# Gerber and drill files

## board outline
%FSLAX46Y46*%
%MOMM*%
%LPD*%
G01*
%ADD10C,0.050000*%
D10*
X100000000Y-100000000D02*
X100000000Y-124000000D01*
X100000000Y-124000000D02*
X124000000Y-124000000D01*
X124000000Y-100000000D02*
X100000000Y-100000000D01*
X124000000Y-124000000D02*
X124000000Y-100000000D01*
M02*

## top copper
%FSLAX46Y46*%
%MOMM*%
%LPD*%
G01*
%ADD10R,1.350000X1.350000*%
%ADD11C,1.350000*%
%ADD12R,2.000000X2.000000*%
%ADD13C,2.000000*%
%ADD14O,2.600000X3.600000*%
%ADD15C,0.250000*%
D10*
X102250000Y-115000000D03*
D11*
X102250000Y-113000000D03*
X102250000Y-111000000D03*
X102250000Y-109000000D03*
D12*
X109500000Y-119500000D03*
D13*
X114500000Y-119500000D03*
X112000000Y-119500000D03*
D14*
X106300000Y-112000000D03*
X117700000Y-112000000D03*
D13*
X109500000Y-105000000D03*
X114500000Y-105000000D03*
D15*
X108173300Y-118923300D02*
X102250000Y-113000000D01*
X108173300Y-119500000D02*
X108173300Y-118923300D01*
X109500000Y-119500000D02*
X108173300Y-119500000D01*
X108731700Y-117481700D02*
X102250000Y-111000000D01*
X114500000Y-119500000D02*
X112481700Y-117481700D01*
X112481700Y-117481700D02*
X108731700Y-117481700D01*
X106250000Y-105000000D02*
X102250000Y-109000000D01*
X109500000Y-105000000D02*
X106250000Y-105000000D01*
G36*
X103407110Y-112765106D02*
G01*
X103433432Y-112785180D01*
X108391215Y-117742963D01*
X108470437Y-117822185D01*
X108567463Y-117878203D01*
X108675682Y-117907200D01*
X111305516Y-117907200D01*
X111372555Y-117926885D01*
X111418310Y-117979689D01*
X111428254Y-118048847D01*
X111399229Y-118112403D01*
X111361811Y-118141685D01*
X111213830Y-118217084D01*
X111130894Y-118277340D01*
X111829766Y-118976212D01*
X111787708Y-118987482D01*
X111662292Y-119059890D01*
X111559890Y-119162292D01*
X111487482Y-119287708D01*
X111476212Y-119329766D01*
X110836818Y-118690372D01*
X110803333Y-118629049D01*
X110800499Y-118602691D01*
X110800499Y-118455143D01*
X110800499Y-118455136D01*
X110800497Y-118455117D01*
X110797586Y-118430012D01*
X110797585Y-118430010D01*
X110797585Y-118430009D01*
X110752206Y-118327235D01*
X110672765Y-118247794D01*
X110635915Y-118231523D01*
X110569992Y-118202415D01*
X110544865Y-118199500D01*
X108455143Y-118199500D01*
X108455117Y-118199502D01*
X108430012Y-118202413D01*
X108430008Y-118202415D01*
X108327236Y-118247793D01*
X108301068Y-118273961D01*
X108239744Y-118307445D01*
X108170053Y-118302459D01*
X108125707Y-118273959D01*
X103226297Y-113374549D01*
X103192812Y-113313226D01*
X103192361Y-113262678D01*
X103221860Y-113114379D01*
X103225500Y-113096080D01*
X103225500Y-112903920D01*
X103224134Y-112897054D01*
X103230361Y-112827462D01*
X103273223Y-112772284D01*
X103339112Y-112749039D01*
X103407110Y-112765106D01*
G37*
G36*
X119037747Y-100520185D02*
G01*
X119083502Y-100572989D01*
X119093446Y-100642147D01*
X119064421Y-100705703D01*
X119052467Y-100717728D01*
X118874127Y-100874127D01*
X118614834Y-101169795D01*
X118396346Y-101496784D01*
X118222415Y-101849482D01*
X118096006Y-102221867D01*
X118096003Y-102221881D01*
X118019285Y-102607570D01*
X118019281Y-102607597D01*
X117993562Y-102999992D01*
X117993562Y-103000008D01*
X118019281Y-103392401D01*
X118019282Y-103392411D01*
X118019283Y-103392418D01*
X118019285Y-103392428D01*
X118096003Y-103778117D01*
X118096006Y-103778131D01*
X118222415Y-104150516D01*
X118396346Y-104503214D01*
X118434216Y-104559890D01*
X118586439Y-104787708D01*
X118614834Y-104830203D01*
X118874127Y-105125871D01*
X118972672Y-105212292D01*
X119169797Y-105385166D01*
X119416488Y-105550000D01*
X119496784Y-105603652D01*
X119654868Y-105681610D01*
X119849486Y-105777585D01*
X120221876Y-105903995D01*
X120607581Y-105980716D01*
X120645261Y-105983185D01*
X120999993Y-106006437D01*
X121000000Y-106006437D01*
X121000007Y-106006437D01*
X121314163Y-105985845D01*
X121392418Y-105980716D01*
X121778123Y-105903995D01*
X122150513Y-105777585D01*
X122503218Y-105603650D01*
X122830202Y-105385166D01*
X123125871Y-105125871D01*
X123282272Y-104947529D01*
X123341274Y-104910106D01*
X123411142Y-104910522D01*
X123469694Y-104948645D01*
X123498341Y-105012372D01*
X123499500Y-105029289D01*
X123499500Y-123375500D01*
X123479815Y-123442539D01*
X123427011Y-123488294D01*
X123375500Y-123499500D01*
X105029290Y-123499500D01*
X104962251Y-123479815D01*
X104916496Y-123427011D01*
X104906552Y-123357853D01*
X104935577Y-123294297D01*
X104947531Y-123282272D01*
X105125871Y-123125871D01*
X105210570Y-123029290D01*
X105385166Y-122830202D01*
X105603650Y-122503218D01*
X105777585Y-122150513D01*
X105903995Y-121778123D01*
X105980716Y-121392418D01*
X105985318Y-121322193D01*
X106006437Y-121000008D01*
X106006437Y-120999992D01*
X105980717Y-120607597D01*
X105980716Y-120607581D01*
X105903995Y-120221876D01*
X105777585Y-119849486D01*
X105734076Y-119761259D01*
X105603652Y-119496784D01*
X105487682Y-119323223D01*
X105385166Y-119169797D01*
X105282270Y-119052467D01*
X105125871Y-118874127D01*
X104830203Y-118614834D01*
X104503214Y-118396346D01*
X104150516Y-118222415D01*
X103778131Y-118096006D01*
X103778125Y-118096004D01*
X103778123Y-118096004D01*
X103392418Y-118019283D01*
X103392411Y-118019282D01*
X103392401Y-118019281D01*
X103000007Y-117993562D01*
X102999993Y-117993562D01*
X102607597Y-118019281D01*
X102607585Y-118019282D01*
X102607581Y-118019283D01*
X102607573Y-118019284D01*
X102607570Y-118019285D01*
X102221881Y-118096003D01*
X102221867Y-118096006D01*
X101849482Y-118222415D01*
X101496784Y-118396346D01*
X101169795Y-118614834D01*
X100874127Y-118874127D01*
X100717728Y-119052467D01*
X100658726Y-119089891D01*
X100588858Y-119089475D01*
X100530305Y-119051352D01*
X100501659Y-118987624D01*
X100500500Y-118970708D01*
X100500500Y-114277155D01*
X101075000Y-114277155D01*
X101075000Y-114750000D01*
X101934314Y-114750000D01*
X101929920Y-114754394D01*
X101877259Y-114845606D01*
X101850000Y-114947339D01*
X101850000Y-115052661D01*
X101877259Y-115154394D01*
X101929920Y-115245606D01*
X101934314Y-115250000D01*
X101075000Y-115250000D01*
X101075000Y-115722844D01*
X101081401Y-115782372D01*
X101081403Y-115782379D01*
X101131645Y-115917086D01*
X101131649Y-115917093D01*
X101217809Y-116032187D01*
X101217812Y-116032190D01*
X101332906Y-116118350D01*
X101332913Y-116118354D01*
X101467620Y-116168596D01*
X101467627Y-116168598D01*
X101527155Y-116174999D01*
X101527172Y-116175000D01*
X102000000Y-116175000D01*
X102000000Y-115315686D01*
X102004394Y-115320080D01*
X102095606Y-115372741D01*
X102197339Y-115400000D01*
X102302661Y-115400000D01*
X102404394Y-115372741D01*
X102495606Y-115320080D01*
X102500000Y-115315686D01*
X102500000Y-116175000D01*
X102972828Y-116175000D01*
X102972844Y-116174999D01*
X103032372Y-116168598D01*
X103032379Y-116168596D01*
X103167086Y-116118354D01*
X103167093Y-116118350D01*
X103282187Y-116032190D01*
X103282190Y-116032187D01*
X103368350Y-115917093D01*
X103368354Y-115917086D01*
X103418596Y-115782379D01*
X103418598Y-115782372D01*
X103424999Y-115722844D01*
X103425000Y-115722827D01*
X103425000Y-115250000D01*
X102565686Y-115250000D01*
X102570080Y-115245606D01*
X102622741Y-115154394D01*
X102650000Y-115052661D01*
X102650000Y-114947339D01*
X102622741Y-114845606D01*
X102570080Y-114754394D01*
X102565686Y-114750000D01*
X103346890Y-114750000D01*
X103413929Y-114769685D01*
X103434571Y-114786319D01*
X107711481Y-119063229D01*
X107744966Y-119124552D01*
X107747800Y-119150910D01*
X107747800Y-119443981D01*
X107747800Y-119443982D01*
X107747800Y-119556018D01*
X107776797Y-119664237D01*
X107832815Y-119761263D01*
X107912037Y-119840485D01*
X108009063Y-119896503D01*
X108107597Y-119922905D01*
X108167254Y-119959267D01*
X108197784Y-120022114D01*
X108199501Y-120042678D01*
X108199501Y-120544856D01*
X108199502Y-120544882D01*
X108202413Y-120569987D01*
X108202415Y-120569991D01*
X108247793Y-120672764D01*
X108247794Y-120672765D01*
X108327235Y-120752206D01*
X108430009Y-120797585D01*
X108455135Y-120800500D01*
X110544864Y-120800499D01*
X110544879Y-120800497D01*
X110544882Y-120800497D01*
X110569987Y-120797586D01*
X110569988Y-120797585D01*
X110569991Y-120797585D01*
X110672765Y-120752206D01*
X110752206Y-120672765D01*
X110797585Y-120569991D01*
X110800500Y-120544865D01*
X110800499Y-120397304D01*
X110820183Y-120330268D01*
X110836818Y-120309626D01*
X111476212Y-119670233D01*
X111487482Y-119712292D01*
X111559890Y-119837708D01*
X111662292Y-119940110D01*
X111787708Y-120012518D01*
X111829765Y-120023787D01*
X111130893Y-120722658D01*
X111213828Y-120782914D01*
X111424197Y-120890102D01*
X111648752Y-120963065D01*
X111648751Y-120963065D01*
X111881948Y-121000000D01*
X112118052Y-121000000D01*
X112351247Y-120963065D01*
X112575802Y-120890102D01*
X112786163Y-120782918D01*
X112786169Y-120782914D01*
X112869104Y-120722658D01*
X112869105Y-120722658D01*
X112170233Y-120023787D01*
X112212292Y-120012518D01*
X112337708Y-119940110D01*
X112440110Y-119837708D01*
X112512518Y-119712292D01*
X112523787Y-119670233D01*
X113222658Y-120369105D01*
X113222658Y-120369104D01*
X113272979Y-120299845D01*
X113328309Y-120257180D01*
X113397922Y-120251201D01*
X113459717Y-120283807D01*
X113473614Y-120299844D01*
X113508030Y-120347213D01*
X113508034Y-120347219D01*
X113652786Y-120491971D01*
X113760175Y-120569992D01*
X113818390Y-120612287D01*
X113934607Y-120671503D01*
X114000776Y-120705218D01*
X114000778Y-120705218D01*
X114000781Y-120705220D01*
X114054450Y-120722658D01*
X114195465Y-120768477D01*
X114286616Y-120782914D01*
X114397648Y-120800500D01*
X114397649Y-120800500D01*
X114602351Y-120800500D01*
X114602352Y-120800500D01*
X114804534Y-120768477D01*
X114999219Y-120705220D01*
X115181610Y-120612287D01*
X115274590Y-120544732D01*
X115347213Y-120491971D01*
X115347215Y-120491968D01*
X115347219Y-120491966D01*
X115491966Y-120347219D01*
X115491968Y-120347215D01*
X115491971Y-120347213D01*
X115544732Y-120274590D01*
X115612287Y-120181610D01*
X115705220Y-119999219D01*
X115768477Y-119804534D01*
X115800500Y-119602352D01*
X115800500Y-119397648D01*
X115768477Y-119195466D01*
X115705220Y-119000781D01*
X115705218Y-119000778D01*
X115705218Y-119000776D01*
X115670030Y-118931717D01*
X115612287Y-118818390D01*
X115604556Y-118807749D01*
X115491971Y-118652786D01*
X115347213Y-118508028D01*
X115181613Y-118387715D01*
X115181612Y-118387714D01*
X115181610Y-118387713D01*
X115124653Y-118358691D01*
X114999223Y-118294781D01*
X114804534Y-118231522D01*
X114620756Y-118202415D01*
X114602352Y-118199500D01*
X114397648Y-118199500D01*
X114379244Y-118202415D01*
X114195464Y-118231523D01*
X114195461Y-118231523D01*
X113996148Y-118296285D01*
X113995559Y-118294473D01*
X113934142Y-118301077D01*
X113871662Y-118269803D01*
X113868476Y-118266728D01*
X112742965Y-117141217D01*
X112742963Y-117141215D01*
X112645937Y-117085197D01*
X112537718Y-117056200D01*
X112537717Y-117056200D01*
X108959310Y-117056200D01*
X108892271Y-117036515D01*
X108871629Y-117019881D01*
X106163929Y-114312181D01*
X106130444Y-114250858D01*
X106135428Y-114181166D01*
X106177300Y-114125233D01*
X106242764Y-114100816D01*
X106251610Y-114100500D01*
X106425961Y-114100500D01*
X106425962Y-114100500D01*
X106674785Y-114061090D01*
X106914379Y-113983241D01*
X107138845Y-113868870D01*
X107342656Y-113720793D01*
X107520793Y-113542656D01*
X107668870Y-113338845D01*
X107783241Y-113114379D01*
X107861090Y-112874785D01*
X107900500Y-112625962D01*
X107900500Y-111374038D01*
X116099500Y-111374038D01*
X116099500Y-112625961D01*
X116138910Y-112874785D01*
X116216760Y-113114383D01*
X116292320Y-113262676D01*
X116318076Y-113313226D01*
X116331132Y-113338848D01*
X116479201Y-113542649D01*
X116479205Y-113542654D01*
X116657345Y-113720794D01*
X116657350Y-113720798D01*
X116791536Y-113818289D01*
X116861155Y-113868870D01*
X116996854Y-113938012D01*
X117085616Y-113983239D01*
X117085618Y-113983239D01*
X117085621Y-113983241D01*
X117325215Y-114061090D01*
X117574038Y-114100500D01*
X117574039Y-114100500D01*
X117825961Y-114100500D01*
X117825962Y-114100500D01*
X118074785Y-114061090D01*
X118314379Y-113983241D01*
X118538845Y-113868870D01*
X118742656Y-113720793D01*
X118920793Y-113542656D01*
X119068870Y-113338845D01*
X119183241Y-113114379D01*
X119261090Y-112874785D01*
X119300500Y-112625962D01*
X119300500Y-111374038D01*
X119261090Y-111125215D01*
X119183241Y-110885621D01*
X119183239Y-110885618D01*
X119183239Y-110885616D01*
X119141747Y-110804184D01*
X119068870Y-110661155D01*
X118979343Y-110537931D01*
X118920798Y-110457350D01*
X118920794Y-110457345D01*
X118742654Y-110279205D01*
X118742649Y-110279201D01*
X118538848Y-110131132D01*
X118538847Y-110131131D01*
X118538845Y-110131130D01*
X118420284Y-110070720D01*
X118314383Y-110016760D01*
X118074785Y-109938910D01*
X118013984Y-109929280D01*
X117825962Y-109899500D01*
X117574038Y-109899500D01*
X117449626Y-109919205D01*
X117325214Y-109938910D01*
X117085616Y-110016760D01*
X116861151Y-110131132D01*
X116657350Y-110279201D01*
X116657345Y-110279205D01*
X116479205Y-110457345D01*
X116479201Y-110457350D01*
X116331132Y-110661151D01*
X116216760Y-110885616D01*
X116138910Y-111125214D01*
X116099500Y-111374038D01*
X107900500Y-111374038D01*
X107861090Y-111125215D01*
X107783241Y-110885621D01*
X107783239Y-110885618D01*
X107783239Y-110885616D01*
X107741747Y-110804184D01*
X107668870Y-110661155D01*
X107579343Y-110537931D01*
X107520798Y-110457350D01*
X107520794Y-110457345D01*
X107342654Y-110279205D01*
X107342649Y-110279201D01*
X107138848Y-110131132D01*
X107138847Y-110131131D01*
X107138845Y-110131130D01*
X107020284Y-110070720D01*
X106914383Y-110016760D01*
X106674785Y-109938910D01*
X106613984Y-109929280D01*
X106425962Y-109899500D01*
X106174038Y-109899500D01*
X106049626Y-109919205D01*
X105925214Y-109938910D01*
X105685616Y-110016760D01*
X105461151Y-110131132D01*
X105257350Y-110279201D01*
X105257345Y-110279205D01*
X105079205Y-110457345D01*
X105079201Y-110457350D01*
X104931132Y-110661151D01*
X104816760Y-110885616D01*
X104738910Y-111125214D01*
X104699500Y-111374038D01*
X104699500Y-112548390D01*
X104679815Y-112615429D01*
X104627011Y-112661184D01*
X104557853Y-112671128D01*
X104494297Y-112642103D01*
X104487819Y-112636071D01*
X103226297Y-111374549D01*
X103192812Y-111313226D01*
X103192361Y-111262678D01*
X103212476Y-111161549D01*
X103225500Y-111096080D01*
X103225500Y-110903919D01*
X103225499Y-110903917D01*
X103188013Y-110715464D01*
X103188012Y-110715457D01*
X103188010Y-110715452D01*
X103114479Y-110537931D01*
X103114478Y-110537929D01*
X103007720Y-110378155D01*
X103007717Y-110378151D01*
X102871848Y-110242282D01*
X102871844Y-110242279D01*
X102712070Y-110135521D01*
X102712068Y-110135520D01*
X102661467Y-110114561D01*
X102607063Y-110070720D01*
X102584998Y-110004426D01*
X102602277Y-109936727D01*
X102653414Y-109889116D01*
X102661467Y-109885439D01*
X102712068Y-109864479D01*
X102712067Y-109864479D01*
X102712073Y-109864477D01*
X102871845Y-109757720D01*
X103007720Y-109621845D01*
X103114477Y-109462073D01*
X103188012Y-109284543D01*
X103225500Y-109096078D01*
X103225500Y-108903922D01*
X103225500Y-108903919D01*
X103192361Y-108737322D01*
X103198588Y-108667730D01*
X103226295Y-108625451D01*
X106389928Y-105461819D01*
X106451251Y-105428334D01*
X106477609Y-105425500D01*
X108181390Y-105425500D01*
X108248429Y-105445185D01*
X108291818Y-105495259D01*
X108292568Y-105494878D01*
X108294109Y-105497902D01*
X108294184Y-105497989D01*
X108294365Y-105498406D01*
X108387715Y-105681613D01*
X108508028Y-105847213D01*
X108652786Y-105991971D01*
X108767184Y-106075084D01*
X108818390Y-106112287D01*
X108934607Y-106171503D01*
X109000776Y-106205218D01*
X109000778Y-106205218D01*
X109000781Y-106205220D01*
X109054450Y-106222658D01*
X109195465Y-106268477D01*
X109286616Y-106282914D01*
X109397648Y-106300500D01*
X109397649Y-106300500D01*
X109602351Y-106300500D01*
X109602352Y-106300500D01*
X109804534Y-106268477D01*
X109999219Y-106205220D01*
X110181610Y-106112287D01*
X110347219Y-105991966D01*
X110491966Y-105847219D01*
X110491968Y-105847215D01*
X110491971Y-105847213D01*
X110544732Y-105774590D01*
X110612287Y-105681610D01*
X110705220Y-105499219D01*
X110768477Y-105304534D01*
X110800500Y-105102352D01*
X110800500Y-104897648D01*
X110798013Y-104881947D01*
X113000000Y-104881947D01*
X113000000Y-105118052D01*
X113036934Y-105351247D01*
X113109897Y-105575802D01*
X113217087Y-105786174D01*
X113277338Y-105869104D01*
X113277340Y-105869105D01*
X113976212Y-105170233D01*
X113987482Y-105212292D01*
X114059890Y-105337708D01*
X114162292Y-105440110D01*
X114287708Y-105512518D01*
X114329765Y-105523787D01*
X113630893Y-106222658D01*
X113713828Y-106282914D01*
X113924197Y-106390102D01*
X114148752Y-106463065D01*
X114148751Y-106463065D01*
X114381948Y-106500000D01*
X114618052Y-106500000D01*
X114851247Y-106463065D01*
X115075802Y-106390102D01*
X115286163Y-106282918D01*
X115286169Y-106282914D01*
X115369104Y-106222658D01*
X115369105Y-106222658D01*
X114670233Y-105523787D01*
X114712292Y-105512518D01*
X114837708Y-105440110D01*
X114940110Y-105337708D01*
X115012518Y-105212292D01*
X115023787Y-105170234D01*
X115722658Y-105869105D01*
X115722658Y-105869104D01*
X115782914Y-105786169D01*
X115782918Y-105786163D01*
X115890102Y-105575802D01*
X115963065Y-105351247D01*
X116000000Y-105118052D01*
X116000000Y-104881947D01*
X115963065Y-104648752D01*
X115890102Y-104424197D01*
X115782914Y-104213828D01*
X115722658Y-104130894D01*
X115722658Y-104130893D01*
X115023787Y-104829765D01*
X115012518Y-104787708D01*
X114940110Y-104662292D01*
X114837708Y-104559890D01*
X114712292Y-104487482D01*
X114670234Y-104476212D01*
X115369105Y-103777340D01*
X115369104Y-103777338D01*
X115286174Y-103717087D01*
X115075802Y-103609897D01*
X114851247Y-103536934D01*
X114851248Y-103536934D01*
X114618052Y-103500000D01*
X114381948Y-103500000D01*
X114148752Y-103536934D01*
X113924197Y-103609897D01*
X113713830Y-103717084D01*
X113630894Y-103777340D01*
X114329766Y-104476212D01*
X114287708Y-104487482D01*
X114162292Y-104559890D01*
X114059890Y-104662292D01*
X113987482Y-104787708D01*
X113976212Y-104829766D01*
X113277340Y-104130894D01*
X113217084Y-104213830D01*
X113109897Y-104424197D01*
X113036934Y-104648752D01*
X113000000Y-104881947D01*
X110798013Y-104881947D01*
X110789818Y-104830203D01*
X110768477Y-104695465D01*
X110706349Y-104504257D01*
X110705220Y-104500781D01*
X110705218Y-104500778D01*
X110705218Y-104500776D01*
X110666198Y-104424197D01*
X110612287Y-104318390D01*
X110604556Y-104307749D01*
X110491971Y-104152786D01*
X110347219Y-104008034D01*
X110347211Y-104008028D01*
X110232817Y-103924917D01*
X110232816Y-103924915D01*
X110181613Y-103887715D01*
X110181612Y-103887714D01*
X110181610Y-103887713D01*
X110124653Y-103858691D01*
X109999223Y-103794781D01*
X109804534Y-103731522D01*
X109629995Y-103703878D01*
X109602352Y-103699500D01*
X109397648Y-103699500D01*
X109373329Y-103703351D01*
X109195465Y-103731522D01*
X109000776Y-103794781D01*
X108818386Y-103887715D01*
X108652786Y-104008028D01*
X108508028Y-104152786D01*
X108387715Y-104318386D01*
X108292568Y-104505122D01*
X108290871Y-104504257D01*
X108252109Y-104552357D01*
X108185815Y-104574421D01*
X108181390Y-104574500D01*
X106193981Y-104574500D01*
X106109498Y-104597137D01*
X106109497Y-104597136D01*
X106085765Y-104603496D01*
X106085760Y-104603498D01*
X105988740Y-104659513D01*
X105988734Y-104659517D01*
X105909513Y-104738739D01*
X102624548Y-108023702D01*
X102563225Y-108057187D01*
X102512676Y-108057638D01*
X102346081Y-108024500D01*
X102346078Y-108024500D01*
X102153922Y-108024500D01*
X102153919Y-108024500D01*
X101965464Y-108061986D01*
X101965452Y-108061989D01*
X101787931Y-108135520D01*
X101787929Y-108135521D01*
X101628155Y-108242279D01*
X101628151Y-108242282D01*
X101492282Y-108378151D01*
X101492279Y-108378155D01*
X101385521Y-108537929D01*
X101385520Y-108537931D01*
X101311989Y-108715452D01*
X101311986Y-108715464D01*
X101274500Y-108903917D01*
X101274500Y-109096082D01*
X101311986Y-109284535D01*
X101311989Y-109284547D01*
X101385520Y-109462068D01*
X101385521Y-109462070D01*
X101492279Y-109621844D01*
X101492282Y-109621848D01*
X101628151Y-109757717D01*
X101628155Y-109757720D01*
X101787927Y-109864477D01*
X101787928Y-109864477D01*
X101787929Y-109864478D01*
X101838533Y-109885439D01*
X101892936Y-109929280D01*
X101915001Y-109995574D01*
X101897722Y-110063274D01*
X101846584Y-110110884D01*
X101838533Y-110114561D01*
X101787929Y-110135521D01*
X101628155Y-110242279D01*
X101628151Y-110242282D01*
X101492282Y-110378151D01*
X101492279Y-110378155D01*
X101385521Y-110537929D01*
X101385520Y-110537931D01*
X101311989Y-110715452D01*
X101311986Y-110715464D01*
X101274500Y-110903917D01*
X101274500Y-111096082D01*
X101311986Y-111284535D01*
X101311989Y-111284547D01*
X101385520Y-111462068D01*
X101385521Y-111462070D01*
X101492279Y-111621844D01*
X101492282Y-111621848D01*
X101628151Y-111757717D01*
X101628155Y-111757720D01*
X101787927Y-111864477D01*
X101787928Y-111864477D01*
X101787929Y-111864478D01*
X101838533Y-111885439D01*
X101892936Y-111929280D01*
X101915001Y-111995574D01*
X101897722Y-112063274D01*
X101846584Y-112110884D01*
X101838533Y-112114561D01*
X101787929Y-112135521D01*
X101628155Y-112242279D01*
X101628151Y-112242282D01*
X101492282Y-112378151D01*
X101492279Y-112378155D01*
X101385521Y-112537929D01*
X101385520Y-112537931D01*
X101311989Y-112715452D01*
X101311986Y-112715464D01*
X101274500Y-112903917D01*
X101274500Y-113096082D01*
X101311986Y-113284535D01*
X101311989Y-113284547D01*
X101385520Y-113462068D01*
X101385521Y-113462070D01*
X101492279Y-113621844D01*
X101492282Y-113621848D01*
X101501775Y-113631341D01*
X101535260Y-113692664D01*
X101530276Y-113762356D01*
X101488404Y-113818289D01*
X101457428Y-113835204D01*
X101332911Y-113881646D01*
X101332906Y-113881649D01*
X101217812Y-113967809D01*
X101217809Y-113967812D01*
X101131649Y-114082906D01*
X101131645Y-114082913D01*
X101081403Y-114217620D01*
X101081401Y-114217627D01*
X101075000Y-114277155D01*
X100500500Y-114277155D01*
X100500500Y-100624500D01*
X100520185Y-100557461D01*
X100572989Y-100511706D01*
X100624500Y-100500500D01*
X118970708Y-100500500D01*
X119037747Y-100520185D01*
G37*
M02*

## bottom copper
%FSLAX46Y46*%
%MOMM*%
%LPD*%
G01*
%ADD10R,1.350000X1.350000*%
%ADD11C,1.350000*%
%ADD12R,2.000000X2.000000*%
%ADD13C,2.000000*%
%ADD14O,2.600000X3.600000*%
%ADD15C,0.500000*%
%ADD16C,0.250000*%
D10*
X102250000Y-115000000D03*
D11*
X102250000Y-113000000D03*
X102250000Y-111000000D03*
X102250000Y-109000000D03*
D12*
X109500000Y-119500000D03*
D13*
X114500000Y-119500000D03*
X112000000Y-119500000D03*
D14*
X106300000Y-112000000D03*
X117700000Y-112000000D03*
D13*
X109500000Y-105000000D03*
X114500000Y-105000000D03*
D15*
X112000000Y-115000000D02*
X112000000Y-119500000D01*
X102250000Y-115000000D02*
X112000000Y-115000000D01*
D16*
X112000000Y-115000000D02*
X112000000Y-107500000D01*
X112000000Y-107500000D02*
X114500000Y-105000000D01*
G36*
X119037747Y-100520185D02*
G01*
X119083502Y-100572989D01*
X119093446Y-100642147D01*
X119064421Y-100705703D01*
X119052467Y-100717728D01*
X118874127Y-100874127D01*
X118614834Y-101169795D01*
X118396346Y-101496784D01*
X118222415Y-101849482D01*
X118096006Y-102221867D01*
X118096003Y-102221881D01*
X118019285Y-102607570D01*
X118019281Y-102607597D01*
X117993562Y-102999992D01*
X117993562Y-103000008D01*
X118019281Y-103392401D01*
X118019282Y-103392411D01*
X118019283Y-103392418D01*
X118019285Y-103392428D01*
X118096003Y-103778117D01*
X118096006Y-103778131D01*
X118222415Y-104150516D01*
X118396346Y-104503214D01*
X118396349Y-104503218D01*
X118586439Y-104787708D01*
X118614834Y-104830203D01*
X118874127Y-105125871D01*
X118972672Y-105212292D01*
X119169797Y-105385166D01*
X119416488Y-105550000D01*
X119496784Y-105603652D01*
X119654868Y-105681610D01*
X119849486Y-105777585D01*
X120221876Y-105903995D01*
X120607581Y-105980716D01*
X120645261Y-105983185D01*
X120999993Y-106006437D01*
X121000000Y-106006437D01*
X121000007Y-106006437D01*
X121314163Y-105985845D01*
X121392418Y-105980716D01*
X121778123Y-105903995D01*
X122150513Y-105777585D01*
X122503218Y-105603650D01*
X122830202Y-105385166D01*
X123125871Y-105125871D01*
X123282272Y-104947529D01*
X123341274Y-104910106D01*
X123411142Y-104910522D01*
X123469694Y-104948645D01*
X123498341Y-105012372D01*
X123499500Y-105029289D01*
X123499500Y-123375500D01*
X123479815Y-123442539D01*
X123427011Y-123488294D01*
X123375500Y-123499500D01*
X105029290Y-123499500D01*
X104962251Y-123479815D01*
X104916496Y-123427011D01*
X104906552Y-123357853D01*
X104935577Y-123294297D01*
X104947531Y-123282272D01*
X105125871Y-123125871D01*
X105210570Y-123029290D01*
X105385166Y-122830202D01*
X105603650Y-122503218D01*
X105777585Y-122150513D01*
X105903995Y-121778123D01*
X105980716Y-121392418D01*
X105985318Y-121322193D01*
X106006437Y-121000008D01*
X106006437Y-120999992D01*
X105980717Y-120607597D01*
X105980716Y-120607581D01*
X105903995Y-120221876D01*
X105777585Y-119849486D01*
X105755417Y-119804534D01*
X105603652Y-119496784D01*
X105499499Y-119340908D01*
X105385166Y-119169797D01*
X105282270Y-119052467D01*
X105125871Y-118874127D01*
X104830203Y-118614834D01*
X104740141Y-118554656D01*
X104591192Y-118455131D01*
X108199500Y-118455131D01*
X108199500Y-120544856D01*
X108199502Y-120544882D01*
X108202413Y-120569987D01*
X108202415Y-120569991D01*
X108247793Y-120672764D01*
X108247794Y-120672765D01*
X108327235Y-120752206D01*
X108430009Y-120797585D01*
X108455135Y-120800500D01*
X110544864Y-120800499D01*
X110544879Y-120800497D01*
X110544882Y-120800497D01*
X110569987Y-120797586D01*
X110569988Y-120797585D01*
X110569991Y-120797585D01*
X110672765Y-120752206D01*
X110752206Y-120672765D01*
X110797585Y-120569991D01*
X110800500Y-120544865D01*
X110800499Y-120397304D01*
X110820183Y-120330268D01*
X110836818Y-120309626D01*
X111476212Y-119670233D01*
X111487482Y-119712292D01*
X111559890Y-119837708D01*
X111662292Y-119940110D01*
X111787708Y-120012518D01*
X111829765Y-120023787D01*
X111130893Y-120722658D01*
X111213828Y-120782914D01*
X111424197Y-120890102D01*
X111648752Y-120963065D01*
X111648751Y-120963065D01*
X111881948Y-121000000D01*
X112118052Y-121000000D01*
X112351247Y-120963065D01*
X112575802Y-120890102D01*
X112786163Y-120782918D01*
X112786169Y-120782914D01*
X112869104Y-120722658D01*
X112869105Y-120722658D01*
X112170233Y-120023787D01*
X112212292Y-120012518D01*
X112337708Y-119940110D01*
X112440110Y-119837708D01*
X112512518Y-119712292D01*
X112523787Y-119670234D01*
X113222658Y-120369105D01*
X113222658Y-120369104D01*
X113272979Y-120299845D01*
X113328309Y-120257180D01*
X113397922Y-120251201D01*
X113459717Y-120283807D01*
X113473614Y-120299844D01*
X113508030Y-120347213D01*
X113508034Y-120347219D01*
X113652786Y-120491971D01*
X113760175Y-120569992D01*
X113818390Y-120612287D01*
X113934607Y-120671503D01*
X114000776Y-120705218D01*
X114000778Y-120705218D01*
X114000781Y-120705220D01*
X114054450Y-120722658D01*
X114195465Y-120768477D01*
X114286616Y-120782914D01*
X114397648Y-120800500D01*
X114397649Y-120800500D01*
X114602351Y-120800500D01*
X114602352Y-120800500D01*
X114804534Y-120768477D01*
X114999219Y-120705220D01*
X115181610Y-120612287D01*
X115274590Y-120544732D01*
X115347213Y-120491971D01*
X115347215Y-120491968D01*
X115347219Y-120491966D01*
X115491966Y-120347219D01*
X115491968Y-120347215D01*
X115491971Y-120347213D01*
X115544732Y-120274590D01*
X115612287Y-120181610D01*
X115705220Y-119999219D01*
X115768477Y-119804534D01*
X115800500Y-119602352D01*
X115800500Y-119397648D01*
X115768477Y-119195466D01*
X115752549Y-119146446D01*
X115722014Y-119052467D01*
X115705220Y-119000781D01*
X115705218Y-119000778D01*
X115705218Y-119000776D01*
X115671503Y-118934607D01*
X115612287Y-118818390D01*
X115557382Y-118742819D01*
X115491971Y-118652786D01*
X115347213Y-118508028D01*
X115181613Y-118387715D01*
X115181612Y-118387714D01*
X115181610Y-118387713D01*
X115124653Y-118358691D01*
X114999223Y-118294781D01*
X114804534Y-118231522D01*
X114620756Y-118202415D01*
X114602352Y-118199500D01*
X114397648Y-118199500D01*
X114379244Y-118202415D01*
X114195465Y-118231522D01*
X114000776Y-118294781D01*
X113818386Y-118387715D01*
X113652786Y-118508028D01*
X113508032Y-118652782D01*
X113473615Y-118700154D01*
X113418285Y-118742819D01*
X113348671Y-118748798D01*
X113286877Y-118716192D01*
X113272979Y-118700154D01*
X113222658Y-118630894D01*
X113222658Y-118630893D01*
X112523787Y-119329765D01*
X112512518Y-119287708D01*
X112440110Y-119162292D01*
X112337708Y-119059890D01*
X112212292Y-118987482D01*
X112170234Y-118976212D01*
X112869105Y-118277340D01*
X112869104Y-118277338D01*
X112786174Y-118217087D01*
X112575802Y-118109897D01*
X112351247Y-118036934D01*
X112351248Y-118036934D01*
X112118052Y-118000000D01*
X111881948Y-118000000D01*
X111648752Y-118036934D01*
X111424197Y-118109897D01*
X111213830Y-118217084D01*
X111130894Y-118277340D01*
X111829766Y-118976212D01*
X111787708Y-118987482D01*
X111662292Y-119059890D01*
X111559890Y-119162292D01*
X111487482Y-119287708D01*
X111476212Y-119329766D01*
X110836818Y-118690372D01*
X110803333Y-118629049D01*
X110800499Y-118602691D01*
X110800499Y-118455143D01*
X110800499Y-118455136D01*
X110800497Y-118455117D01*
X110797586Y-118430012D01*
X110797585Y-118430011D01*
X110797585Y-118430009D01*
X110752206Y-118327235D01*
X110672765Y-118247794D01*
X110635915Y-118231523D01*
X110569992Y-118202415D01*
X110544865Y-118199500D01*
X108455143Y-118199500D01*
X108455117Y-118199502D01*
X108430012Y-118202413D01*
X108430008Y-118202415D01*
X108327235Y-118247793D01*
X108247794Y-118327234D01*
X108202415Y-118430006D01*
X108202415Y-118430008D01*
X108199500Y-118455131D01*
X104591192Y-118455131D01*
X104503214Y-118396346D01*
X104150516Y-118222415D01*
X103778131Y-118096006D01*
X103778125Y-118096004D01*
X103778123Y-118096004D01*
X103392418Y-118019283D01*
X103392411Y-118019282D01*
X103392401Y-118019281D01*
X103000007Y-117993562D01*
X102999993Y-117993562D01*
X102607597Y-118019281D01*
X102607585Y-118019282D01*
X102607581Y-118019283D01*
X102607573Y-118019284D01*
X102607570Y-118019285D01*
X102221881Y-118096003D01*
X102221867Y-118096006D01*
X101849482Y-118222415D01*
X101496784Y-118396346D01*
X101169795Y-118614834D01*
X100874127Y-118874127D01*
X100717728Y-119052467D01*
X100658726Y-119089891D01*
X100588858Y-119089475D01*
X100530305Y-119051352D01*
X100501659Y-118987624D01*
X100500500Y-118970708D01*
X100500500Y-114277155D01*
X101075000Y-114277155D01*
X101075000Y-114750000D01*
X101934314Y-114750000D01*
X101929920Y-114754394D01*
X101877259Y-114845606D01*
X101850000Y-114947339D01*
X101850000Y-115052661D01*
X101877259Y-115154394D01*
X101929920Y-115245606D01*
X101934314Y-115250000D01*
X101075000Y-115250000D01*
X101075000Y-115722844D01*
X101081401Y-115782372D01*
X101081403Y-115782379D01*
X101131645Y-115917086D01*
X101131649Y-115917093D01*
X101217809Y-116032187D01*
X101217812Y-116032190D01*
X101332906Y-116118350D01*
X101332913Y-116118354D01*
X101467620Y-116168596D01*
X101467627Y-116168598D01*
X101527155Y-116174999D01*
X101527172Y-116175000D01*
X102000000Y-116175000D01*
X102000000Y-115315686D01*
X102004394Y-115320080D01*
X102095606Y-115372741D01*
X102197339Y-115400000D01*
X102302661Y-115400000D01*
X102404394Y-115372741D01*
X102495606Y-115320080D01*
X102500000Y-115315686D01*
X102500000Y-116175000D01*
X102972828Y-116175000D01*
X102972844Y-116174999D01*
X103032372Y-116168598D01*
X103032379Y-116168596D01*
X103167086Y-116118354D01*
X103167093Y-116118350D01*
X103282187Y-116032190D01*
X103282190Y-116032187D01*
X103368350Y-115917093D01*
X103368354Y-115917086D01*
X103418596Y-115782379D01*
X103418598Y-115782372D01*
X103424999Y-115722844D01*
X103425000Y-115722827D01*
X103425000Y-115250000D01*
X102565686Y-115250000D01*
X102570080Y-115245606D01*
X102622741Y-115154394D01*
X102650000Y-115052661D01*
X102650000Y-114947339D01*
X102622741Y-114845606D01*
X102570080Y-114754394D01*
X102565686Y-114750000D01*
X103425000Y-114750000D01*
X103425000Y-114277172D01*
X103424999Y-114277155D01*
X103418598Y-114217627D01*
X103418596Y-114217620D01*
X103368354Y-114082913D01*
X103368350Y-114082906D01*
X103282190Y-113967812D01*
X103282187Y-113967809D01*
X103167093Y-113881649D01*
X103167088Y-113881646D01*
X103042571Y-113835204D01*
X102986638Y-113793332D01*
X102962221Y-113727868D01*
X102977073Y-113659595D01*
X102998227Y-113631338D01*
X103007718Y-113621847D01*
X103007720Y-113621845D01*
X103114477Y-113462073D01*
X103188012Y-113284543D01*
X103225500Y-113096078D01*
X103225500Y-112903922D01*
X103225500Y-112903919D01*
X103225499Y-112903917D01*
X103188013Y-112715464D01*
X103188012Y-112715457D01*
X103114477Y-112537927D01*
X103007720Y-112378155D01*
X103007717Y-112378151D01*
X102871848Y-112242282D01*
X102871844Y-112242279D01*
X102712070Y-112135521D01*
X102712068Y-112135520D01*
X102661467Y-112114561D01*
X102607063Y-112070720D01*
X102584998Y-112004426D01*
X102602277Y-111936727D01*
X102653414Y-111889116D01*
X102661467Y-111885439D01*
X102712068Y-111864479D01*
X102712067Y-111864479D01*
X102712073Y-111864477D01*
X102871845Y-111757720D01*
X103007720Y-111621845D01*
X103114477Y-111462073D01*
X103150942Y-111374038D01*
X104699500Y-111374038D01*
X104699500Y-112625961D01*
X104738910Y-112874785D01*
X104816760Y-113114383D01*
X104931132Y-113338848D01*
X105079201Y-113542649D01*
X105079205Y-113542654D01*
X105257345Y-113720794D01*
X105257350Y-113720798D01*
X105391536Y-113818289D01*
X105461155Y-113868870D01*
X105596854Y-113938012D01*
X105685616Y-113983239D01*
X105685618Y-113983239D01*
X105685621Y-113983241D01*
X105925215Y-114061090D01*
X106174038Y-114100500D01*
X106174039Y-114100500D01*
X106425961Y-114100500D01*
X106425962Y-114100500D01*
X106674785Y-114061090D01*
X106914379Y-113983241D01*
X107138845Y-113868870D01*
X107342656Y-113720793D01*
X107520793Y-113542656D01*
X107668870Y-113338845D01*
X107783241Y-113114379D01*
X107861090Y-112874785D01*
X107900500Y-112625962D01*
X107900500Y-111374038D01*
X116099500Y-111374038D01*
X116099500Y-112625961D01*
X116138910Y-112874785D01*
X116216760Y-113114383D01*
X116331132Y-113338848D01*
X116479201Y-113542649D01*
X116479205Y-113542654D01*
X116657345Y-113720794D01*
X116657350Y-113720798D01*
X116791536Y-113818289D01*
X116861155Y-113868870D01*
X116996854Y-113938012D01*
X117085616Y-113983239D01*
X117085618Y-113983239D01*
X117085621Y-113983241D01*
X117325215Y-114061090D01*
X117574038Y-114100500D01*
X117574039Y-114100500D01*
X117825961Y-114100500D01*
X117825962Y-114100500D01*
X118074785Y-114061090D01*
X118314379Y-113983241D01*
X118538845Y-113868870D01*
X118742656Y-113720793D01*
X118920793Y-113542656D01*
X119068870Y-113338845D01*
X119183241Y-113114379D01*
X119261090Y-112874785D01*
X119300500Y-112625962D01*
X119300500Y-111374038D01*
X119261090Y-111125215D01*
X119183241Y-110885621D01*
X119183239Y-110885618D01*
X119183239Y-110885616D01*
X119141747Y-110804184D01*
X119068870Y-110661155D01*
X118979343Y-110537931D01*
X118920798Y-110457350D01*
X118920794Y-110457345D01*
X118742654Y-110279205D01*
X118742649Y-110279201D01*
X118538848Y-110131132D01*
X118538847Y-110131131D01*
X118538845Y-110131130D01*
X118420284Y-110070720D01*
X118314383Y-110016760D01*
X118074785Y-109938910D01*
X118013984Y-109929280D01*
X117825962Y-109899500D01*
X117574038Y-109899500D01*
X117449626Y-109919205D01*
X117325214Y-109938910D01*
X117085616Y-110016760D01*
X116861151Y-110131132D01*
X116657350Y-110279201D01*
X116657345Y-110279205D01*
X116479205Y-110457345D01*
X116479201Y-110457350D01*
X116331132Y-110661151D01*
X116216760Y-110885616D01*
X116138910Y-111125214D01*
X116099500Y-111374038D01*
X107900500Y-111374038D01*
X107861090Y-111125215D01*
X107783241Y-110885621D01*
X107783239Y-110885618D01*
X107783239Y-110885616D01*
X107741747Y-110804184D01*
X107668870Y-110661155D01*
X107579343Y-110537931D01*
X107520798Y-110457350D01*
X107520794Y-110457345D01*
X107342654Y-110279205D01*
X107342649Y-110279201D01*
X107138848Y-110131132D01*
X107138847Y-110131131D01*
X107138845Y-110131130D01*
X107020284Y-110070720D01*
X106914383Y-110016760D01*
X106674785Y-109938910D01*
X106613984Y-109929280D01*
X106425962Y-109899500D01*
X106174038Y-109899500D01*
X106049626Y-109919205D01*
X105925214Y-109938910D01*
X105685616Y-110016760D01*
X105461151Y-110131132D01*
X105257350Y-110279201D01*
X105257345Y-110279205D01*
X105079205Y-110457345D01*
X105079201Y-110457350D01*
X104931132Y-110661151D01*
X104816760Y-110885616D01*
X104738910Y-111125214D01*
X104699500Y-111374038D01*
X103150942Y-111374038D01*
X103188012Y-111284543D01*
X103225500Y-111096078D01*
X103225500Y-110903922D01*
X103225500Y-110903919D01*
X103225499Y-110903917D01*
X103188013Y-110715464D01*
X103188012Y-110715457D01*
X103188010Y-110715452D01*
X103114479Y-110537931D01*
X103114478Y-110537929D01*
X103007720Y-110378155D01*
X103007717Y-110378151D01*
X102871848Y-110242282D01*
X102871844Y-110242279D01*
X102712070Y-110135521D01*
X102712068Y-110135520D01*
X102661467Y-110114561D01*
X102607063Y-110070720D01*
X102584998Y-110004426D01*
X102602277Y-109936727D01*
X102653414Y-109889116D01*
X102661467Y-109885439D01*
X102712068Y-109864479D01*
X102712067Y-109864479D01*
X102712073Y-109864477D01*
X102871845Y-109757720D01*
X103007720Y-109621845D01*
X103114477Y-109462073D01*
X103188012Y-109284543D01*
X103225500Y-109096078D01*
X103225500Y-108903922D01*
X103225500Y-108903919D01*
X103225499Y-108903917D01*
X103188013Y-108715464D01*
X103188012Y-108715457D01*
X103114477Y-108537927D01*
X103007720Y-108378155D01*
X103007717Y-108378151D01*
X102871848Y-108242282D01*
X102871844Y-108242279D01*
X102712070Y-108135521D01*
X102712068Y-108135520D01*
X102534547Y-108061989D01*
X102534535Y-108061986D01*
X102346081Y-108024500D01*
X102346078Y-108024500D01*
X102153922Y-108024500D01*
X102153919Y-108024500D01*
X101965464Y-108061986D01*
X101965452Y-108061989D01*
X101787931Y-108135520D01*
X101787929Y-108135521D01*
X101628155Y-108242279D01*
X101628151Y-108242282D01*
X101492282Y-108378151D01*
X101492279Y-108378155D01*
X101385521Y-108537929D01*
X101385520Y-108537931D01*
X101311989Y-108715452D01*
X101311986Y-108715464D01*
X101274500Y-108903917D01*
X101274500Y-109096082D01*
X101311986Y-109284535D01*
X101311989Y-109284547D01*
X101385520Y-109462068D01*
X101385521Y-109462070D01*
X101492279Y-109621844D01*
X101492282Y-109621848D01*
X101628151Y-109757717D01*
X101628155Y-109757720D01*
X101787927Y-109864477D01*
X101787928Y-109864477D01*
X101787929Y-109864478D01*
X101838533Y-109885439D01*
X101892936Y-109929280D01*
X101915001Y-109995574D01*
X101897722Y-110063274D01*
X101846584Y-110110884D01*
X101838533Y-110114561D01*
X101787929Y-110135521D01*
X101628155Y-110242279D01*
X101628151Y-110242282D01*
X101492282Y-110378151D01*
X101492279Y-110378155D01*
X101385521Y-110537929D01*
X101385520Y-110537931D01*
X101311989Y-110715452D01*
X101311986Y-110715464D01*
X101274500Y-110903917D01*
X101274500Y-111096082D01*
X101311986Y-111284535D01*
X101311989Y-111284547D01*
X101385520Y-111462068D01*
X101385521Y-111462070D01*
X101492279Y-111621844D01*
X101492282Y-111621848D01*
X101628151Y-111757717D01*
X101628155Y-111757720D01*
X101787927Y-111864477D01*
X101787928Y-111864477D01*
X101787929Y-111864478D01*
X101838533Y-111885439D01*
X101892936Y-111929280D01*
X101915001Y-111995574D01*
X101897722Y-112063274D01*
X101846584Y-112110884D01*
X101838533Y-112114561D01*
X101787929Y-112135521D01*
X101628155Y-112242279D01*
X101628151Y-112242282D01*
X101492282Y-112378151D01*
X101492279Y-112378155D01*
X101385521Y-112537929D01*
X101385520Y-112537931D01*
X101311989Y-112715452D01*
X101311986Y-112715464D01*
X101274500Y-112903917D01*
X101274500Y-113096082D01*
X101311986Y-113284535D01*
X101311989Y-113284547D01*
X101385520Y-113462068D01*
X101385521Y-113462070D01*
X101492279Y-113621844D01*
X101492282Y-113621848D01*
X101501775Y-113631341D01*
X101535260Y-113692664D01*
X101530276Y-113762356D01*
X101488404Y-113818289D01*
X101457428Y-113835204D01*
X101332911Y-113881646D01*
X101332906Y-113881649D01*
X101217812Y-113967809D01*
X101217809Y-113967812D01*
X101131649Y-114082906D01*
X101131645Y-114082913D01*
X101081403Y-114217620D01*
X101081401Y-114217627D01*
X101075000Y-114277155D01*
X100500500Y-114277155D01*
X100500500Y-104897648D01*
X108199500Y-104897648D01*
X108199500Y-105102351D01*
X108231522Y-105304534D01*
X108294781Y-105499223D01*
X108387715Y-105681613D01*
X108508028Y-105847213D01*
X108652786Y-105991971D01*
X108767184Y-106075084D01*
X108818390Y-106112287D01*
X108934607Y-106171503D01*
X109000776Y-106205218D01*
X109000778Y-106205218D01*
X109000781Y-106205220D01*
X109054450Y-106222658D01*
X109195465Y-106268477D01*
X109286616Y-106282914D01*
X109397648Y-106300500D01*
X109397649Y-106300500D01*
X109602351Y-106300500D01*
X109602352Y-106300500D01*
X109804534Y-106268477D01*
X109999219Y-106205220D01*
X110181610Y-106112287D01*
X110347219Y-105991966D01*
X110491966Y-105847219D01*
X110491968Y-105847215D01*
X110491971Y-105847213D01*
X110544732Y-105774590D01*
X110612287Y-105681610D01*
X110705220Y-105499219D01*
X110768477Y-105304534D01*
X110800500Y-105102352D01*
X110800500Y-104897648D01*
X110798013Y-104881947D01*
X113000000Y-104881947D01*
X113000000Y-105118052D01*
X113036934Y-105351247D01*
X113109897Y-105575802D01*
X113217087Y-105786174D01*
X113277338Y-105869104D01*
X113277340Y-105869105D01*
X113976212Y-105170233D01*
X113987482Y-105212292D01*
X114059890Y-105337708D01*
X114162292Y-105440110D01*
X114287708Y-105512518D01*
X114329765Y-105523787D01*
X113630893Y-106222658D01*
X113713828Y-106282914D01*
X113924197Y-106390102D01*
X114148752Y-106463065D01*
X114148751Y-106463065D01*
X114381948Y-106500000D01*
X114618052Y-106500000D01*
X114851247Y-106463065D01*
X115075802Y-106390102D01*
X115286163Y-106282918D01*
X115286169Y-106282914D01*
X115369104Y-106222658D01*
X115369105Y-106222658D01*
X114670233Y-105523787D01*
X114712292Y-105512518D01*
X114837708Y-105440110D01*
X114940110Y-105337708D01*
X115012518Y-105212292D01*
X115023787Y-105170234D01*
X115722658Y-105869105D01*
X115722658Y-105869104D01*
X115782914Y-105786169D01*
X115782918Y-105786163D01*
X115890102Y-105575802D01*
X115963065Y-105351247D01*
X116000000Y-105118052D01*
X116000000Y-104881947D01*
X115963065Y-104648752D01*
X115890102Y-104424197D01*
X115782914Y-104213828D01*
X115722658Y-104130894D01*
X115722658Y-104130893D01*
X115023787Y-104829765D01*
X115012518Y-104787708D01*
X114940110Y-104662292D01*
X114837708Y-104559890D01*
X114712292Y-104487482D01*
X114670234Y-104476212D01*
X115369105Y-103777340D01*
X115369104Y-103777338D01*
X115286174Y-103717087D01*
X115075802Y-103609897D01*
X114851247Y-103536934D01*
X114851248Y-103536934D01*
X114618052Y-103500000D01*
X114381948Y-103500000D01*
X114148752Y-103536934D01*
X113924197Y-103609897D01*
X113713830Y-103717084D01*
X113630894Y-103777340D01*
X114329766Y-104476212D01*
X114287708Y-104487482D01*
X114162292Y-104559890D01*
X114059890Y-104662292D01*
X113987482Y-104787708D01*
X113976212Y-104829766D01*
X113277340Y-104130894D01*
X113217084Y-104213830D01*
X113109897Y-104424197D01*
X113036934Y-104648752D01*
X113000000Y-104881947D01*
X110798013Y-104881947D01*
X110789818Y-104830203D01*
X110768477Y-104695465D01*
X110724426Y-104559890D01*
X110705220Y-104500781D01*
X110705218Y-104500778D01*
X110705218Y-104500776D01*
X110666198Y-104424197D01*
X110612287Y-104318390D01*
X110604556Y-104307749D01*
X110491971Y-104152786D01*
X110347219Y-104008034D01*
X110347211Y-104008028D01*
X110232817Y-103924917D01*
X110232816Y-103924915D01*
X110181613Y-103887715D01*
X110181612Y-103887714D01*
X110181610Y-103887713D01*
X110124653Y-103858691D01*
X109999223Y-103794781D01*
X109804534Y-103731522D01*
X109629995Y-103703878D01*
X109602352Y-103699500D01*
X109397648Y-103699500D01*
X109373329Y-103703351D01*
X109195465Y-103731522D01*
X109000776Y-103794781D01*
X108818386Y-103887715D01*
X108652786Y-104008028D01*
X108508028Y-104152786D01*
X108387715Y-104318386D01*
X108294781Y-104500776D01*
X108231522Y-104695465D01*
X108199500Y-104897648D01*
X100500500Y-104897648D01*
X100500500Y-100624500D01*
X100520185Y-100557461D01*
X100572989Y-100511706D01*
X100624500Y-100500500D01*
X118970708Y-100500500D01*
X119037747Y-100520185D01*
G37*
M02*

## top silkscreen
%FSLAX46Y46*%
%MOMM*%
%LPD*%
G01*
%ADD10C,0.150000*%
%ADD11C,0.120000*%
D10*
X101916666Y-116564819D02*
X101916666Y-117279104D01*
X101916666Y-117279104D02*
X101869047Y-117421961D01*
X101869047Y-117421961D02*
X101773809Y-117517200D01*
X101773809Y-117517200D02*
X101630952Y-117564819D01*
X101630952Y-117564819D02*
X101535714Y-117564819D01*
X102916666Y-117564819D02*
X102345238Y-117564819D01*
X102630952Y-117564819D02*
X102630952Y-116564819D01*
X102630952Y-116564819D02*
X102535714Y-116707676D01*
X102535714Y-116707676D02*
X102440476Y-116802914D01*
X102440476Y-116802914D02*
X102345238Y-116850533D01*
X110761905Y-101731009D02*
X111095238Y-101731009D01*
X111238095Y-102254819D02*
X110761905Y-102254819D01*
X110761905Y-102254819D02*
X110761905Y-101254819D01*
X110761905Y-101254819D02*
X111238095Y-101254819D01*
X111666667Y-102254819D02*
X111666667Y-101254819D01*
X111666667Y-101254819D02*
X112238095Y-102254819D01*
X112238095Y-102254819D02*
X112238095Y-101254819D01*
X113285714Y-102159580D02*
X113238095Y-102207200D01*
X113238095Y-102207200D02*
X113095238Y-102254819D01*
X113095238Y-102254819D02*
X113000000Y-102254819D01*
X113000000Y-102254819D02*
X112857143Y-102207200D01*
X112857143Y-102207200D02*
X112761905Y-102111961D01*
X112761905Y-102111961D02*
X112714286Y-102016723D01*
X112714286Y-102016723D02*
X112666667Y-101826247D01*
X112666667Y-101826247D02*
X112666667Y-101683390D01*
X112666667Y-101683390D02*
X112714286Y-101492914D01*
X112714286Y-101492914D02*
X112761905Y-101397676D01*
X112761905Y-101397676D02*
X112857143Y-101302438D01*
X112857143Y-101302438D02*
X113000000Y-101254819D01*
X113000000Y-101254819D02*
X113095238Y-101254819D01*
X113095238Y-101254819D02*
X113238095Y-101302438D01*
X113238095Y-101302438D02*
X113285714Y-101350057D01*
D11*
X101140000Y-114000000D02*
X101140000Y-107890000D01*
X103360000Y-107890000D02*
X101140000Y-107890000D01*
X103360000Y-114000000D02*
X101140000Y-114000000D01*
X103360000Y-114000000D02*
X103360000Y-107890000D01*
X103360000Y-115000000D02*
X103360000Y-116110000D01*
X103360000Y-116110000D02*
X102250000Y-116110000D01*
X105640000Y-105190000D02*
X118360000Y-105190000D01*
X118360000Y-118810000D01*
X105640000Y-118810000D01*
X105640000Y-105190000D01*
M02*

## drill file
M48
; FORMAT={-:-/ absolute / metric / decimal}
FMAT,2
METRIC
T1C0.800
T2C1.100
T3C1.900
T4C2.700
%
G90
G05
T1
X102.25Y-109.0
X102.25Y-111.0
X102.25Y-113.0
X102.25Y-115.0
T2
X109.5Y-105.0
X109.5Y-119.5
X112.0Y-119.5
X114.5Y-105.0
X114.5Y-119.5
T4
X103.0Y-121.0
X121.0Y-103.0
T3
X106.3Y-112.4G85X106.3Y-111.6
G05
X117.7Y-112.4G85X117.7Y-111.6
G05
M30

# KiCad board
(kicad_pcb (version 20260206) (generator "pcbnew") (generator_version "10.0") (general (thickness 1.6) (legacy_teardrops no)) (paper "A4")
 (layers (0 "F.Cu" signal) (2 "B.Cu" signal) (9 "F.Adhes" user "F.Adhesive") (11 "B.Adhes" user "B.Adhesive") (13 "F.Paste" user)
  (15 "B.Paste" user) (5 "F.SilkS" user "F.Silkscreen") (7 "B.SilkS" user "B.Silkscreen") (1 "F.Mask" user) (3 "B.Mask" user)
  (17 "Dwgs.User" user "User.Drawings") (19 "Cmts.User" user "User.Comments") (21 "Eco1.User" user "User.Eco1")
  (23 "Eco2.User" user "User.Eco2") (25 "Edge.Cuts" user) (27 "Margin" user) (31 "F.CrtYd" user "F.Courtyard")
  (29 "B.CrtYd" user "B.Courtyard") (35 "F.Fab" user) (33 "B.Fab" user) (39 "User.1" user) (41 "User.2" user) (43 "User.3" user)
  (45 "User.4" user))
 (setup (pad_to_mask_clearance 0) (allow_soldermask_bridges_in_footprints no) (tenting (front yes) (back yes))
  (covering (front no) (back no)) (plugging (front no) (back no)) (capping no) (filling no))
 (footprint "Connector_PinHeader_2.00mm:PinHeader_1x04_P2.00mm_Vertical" (layer "F.Cu") (at 102.25 115 180)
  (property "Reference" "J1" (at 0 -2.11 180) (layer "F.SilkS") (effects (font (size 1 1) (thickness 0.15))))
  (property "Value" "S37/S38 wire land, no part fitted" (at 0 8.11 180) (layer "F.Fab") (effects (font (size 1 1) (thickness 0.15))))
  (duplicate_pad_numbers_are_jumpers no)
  (fp_line (start 1.11 1) (end 1.11 7.11) (stroke (width 0.12) (type solid)) (layer "F.SilkS"))
  (fp_line (start -1.11 7.11) (end 1.11 7.11) (stroke (width 0.12) (type solid)) (layer "F.SilkS"))
  (fp_line (start -1.11 1) (end 1.11 1) (stroke (width 0.12) (type solid)) (layer "F.SilkS"))
  (fp_line (start -1.11 1) (end -1.11 7.11) (stroke (width 0.12) (type solid)) (layer "F.SilkS"))
  (fp_line (start -1.11 0) (end -1.11 -1.11) (stroke (width 0.12) (type solid)) (layer "F.SilkS"))
  (fp_line (start -1.11 -1.11) (end 0 -1.11) (stroke (width 0.12) (type solid)) (layer "F.SilkS"))
  (pad "1" thru_hole rect (at 0 0 180) (size 1.35 1.35) (drill 0.8) (layers "*.Cu" "*.Mask") (remove_unused_layers no) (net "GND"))
  (pad "2" thru_hole circle (at 0 2 180) (size 1.35 1.35) (drill 0.8) (layers "*.Cu" "*.Mask") (remove_unused_layers no) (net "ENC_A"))
  (pad "3" thru_hole circle (at 0 4 180) (size 1.35 1.35) (drill 0.8) (layers "*.Cu" "*.Mask") (remove_unused_layers no) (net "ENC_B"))
  (pad "4" thru_hole circle (at 0 6 180) (size 1.35 1.35) (drill 0.8) (layers "*.Cu" "*.Mask") (remove_unused_layers no) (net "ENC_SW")))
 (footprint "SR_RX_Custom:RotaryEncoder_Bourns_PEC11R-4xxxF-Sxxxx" (layer "F.Cu") (at 109.5 119.5 90)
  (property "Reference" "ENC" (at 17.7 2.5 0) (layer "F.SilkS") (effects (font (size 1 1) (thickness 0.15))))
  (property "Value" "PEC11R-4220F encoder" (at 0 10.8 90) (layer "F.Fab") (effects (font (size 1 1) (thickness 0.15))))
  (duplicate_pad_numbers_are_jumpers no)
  (fp_rect (start 0.69 -3.86) (end 14.31 8.86) (stroke (width 0.12) (type solid)) (fill no) (layer "F.SilkS"))
  (pad "A" thru_hole rect (at 0 0 90) (size 2 2) (drill 1.1) (layers "*.Cu" "*.Mask") (remove_unused_layers no) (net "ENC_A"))
  (pad "B" thru_hole circle (at 0 5 90) (size 2 2) (drill 1.1) (layers "*.Cu" "*.Mask") (remove_unused_layers no) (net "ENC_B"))
  (pad "C" thru_hole circle (at 0 2.5 90) (size 2 2) (drill 1.1) (layers "*.Cu" "*.Mask") (remove_unused_layers no) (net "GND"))
  (pad "MP" thru_hole oval (at 7.5 -3.2 90) (size 3.6 2.6) (drill oval 2.7 1.9) (layers "*.Cu" "*.Mask") (remove_unused_layers no))
  (pad "MP" thru_hole oval (at 7.5 8.2 90) (size 3.6 2.6) (drill oval 2.7 1.9) (layers "*.Cu" "*.Mask") (remove_unused_layers no))
  (pad "S1" thru_hole circle (at 14.5 0 90) (size 2 2) (drill 1.1) (layers "*.Cu" "*.Mask") (remove_unused_layers no) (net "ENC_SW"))
  (pad "S2" thru_hole circle (at 14.5 5 90) (size 2 2) (drill 1.1) (layers "*.Cu" "*.Mask") (remove_unused_layers no) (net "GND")))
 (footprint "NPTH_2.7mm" (layer "F.Cu") (at 103 121)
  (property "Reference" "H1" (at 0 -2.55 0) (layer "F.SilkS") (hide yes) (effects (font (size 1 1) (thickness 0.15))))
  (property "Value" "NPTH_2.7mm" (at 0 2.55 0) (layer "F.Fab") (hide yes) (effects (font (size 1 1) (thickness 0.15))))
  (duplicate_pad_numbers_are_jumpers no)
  (pad "" np_thru_hole circle (at 0 0) (size 2.7 2.7) (drill 2.7) (layers "*.Cu" "*.Mask")))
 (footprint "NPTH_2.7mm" (layer "F.Cu") (at 121 103)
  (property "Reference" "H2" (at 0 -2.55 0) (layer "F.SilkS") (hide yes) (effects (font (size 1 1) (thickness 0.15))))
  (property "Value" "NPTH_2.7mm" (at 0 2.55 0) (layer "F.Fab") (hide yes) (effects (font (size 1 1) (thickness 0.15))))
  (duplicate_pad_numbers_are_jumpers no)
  (pad "" np_thru_hole circle (at 0 0) (size 2.7 2.7) (drill 2.7) (layers "*.Cu" "*.Mask")))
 (gr_line (start 100 100) (end 100 124) (stroke (width 0.05) (type default)) (layer "Edge.Cuts"))
 (gr_line (start 100 124) (end 124 124) (stroke (width 0.05) (type default)) (layer "Edge.Cuts"))
 (gr_line (start 124 100) (end 100 100) (stroke (width 0.05) (type default)) (layer "Edge.Cuts"))
 (gr_line (start 124 124) (end 124 100) (stroke (width 0.05) (type default)) (layer "Edge.Cuts"))
 (segment (start 112 115) (end 112 119.5) (width 0.5) (locked yes) (layer "B.Cu") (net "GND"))
 (segment (start 102.25 115) (end 112 115) (width 0.5) (locked yes) (layer "B.Cu") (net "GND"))
 (segment (start 112 115) (end 112 107.5) (width 0.25) (layer "B.Cu") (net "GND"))
 (segment (start 112 107.5) (end 114.5 105) (width 0.25) (layer "B.Cu") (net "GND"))
 (segment (start 108.1733 118.9233) (end 102.25 113) (width 0.25) (layer "F.Cu") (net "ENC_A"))
 (segment (start 108.1733 119.5) (end 108.1733 118.9233) (width 0.25) (layer "F.Cu") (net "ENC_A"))
 (segment (start 109.5 119.5) (end 108.1733 119.5) (width 0.25) (layer "F.Cu") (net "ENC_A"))
 (segment (start 108.7317 117.4817) (end 102.25 111) (width 0.25) (layer "F.Cu") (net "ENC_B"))
 (segment (start 114.5 119.5) (end 112.4817 117.4817) (width 0.25) (layer "F.Cu") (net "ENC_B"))
 (segment (start 112.4817 117.4817) (end 108.7317 117.4817) (width 0.25) (layer "F.Cu") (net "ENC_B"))
 (segment (start 106.25 105) (end 102.25 109) (width 0.25) (layer "F.Cu") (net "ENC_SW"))
 (segment (start 109.5 105) (end 106.25 105) (width 0.25) (layer "F.Cu") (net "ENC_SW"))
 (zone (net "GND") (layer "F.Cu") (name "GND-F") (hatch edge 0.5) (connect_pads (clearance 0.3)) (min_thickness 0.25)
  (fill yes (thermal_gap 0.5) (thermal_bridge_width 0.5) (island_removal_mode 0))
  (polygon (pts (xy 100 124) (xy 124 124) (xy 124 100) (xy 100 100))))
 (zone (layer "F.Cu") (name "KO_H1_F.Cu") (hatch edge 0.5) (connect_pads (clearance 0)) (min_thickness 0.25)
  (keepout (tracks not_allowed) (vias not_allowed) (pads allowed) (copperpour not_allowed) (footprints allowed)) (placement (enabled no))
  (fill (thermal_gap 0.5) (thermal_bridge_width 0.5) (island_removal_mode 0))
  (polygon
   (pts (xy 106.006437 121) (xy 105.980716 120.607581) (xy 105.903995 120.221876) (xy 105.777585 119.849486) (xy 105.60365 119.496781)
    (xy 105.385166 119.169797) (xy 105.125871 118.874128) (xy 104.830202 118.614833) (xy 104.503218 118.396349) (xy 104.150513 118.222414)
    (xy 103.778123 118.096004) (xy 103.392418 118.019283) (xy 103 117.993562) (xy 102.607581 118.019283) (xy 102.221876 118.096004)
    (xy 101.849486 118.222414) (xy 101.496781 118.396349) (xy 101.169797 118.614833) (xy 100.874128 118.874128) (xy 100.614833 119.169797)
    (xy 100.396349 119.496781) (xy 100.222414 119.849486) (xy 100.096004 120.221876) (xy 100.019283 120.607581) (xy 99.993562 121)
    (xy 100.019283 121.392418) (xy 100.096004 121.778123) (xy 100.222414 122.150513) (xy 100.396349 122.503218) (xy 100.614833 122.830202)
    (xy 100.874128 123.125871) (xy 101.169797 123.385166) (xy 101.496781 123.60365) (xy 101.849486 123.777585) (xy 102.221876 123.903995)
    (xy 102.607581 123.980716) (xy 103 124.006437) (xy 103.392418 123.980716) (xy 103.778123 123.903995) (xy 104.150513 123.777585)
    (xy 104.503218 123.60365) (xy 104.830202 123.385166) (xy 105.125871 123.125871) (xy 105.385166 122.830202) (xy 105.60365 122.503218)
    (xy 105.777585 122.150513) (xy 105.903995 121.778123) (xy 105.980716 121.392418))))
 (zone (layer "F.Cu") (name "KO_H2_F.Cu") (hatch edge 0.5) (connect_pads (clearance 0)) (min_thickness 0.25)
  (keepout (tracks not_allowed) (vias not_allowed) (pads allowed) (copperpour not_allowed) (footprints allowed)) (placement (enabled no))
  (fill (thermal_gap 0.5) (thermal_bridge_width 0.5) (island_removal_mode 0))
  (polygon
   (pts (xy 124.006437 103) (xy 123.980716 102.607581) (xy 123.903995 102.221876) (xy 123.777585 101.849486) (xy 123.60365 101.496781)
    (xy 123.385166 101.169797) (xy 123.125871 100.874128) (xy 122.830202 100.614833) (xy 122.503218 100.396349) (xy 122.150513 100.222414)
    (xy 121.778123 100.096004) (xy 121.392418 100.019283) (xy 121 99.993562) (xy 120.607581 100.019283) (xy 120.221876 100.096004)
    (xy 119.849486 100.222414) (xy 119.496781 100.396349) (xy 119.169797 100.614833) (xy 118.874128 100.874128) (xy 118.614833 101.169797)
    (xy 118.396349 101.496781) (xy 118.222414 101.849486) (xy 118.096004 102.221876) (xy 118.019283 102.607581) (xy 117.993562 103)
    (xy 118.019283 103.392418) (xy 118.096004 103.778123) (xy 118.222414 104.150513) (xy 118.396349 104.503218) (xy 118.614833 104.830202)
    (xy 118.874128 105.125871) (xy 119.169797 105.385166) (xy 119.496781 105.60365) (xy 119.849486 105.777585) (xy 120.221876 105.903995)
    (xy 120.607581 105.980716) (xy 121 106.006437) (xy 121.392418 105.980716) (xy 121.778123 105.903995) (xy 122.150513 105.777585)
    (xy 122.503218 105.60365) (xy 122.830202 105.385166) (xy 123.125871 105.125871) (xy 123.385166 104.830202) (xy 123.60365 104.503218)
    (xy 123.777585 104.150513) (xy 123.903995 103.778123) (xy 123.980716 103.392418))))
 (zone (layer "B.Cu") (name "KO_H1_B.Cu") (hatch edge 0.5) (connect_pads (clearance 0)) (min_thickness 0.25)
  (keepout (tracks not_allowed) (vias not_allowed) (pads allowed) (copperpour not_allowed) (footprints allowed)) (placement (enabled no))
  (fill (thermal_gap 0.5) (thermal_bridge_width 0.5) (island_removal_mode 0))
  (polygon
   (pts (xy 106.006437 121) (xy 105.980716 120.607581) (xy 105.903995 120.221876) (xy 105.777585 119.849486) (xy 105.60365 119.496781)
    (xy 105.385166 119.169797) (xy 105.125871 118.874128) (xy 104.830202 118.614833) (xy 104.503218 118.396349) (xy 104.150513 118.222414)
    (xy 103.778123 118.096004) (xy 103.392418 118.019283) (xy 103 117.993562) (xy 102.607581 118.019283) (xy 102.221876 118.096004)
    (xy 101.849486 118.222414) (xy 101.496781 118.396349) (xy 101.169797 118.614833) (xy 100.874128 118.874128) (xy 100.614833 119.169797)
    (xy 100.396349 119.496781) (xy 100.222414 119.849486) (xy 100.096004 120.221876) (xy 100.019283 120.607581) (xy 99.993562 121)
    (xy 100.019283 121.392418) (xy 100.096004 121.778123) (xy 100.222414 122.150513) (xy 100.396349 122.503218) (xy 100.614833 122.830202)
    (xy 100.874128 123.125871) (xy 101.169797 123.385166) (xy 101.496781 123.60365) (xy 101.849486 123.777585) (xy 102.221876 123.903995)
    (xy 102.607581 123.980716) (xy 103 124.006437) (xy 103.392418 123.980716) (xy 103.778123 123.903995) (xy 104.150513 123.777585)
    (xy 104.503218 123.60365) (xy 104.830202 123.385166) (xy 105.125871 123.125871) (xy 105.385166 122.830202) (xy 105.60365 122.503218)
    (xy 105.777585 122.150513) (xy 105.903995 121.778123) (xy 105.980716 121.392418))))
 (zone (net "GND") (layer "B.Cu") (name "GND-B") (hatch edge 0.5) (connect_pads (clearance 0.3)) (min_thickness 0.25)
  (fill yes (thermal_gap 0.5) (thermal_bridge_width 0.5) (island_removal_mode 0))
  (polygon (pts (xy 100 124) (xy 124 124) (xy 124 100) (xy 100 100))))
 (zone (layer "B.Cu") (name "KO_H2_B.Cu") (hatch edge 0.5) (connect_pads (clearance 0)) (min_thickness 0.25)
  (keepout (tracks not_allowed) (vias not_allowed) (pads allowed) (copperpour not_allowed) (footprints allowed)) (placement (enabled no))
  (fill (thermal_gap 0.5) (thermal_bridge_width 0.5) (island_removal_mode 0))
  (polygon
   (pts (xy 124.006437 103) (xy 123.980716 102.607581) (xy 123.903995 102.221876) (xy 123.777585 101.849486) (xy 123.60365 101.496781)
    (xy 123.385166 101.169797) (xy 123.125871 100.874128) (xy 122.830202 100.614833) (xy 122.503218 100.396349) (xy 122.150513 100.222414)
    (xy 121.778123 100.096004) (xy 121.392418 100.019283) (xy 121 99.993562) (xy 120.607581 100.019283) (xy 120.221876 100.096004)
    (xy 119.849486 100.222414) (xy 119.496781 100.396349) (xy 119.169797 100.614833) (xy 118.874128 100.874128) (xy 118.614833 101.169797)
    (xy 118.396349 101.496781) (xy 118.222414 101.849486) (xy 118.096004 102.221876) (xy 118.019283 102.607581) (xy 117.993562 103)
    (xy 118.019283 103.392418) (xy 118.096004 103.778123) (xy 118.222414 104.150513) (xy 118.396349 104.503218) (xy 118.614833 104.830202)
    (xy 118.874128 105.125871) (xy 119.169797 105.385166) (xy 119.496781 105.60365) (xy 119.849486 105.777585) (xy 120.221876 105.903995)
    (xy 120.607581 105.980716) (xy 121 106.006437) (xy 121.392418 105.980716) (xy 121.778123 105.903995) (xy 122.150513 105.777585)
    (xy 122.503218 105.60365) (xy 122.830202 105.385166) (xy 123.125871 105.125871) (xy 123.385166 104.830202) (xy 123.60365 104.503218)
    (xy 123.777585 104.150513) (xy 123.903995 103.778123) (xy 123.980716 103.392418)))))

